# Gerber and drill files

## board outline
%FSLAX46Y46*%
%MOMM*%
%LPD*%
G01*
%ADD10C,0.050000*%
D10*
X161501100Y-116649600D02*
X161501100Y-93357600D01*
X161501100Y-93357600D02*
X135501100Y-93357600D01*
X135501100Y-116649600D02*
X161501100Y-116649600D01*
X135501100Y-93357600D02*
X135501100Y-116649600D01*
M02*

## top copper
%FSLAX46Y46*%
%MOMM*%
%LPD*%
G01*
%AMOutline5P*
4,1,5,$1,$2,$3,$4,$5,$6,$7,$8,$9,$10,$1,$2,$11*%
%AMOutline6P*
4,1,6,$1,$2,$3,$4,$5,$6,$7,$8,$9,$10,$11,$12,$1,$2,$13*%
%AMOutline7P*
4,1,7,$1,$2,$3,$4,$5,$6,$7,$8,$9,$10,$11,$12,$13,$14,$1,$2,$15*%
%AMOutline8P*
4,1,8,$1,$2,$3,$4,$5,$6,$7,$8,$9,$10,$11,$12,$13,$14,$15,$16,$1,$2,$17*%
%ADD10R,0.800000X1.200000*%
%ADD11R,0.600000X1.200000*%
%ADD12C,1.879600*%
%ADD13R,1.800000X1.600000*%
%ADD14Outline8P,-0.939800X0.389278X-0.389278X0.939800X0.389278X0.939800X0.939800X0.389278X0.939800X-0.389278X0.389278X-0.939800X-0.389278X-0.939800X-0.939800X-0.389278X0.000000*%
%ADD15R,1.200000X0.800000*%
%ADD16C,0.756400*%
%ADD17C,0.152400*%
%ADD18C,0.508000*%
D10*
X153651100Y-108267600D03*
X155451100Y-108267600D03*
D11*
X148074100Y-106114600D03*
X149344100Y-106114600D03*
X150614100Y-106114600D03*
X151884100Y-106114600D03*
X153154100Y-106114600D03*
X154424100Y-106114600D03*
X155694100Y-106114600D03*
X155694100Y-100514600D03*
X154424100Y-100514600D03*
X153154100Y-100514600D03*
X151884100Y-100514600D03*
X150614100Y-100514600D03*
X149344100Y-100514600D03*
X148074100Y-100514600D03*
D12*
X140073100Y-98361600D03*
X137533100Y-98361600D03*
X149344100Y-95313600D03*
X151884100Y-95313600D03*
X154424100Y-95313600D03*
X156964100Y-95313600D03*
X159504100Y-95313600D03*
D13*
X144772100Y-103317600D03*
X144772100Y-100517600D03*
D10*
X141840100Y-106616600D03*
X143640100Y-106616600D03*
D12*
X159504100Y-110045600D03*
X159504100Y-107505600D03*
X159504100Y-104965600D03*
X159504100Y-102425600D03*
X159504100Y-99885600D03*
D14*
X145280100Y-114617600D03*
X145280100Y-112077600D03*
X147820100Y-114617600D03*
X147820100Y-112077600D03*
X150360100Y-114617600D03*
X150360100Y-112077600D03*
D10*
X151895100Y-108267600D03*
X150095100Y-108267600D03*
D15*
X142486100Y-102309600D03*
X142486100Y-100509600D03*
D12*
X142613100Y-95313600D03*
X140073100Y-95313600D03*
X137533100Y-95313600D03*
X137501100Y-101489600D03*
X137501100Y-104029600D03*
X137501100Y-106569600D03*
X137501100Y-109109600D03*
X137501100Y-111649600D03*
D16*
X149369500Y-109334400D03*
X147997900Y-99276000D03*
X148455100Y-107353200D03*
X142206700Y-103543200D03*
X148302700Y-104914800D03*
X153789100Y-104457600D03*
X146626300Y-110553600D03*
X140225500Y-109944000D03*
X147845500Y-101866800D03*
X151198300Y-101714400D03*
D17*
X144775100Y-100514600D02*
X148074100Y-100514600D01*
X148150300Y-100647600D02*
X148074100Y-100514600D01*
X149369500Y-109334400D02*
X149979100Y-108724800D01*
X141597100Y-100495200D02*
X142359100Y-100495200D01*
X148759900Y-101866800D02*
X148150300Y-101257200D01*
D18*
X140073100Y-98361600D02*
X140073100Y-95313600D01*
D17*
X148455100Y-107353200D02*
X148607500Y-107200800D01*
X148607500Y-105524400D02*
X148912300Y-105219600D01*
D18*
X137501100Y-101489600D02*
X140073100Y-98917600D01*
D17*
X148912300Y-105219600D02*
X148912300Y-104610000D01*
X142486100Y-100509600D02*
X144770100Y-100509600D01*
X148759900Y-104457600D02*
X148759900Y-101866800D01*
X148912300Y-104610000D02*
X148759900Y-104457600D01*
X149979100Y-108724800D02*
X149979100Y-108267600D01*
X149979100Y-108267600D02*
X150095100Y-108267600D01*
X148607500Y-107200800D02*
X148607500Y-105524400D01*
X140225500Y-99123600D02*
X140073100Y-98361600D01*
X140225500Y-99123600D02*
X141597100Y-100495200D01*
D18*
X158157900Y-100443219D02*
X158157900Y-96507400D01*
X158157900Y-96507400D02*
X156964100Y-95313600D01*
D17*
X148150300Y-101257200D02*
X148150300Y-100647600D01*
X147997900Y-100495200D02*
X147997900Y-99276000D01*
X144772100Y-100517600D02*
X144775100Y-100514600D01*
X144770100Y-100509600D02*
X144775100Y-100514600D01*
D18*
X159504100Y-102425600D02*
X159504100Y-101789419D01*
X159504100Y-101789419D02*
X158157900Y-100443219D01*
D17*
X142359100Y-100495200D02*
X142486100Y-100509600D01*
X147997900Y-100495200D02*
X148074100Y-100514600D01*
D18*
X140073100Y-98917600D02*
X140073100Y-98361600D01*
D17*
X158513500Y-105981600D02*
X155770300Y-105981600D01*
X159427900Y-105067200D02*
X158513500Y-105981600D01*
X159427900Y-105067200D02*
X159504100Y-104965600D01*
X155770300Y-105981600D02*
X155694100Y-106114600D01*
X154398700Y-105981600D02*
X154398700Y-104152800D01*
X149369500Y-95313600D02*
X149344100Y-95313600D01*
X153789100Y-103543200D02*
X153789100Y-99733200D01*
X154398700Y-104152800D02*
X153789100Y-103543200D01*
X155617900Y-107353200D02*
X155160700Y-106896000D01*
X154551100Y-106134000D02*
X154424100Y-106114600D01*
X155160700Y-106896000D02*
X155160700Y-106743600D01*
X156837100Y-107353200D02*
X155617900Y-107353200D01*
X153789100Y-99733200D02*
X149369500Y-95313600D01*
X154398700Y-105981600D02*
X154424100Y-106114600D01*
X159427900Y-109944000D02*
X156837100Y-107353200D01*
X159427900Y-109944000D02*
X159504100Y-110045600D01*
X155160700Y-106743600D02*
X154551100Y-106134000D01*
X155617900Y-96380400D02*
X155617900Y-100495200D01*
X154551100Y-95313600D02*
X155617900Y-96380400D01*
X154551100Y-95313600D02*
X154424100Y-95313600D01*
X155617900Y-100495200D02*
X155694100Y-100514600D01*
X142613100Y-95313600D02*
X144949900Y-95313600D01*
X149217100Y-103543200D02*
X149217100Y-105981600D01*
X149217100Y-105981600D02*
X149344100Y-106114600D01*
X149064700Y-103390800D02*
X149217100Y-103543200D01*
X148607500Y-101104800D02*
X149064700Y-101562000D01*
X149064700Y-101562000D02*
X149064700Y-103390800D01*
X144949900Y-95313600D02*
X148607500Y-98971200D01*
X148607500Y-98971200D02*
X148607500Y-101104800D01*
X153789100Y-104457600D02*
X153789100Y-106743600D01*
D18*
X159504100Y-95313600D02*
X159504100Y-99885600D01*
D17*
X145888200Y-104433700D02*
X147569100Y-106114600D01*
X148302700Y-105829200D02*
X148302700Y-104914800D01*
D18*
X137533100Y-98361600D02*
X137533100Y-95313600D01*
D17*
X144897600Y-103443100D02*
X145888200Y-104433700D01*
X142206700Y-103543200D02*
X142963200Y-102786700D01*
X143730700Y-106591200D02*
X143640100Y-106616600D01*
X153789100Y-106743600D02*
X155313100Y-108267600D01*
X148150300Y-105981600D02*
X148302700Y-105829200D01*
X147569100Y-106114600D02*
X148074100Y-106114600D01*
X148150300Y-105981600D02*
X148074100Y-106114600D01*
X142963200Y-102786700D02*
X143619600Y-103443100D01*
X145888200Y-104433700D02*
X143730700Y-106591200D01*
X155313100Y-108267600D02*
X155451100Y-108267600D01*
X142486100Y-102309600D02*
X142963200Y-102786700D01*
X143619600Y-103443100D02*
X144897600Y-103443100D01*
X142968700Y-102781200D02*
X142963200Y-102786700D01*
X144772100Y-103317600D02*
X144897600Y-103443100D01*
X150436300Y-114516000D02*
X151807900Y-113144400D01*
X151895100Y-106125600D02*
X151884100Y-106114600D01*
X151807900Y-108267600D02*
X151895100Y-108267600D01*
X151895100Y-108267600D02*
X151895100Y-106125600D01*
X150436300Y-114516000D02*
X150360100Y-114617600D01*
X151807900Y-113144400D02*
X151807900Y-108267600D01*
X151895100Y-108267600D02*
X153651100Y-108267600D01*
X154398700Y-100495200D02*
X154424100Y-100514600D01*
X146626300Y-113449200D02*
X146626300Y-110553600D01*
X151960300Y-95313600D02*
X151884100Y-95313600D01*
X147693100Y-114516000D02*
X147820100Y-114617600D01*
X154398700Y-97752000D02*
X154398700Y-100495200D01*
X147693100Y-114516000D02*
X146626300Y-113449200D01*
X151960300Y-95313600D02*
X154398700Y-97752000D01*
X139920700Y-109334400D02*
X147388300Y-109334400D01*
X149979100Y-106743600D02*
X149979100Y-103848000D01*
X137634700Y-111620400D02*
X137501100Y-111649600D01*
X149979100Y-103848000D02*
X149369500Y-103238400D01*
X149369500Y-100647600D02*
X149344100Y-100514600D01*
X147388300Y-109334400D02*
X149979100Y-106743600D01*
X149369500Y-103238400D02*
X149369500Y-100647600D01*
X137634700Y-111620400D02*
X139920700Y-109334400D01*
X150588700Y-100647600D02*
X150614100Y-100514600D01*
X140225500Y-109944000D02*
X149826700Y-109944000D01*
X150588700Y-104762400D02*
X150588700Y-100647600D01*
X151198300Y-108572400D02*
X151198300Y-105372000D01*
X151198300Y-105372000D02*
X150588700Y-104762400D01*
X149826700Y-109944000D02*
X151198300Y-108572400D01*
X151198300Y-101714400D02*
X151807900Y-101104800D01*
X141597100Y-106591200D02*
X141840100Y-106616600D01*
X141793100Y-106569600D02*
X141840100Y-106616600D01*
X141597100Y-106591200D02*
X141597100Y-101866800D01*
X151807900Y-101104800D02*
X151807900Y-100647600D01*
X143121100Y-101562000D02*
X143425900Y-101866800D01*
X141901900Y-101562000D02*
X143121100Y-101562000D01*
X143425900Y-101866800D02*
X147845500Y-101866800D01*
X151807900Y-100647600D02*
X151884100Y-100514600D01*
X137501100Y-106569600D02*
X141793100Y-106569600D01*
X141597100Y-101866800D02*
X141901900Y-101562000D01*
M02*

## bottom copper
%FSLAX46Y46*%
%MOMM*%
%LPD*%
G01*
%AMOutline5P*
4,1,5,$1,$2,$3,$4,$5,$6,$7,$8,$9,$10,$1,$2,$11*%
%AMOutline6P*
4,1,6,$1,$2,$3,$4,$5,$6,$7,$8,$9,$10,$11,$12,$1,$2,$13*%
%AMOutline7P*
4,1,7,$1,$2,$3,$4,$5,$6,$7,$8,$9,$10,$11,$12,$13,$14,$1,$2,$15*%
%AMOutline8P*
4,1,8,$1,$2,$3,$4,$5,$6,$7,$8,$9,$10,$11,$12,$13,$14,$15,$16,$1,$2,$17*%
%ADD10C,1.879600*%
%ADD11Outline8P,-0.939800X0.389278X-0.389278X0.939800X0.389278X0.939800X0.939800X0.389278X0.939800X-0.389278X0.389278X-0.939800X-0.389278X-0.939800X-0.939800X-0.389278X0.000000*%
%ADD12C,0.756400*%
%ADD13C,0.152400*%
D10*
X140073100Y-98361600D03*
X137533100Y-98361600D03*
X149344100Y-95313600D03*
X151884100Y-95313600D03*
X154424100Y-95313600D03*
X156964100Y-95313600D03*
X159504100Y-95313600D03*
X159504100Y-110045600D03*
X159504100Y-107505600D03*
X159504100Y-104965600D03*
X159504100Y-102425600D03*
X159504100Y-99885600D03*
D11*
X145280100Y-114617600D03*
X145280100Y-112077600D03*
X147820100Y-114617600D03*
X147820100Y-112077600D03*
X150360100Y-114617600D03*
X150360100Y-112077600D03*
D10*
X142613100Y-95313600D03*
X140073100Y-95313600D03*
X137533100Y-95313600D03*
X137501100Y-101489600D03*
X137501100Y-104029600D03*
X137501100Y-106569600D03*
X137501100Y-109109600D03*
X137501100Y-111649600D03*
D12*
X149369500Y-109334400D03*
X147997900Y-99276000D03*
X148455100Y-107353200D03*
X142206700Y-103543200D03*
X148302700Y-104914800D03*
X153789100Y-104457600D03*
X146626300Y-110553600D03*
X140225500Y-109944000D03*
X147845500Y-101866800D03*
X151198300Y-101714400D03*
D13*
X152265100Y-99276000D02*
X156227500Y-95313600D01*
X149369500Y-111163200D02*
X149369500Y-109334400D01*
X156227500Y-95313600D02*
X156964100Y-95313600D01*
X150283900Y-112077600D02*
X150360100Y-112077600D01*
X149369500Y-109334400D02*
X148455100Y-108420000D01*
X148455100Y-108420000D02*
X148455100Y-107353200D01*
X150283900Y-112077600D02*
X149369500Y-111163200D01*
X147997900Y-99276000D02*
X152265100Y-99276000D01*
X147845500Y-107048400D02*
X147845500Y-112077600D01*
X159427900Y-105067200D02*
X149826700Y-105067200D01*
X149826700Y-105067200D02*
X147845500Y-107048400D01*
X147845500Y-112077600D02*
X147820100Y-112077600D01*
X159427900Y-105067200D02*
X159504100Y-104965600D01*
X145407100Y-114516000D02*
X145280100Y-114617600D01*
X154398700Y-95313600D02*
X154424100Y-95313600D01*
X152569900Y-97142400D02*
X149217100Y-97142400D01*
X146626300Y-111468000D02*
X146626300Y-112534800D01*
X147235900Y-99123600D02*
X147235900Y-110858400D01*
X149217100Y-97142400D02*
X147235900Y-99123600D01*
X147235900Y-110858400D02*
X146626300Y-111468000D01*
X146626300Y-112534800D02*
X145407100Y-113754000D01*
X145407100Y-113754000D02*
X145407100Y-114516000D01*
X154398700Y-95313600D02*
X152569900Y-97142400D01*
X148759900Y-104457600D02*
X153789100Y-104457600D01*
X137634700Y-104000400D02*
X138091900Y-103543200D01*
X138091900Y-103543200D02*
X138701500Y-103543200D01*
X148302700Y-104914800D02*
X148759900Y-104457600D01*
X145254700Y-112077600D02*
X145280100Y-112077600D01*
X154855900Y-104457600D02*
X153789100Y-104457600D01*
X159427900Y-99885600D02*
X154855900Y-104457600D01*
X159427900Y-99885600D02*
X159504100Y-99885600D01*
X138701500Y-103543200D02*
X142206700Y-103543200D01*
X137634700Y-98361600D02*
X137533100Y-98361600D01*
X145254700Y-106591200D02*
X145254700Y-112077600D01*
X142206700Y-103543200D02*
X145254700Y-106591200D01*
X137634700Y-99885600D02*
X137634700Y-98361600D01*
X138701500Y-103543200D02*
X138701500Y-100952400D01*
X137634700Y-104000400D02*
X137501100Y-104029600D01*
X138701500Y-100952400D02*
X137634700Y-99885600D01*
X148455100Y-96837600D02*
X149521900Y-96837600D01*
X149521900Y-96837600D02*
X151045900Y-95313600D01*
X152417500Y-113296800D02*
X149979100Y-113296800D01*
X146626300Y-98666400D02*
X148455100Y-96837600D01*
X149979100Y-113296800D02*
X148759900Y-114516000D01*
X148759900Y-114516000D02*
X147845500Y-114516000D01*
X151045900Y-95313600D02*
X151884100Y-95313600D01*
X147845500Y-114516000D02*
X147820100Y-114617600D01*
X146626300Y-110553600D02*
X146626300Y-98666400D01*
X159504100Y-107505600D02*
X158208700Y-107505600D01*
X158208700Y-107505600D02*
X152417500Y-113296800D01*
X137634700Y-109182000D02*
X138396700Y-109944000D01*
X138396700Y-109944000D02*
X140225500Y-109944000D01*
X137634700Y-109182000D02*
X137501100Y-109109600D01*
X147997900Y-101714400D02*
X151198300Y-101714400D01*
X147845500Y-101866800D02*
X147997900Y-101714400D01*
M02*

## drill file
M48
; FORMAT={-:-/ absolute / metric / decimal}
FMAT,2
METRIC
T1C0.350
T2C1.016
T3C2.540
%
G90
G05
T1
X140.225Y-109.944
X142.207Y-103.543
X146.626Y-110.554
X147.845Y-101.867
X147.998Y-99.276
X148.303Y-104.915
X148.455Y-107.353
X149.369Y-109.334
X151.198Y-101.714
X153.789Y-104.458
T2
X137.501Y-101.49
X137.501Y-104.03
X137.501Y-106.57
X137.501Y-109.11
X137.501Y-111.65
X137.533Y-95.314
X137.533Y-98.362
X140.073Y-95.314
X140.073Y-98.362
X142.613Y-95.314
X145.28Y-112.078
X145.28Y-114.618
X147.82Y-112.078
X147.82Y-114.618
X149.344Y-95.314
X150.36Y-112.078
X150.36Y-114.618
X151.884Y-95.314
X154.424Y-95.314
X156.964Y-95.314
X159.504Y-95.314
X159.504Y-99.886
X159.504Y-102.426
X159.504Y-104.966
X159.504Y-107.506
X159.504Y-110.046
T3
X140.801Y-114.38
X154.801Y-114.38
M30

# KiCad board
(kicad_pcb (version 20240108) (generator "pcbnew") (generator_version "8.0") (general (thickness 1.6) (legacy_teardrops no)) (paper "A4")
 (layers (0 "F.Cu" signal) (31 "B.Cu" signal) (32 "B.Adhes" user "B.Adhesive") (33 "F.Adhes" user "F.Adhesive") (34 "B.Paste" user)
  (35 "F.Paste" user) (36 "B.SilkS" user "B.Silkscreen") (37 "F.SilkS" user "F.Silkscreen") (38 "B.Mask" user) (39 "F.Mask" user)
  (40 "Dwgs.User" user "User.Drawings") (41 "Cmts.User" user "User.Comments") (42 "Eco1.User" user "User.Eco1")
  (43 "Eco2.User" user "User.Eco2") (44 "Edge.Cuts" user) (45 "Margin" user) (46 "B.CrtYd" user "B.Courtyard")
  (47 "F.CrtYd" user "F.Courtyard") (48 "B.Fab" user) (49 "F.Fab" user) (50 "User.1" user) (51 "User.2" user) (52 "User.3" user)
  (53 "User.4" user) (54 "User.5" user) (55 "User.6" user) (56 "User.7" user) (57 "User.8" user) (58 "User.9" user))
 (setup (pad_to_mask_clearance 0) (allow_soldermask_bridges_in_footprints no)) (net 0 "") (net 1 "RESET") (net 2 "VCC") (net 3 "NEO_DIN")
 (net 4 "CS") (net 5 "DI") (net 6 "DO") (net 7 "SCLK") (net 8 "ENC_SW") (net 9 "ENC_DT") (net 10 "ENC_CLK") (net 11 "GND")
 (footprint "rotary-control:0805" (layer "F.Cu") (at 154.5511 108.2676)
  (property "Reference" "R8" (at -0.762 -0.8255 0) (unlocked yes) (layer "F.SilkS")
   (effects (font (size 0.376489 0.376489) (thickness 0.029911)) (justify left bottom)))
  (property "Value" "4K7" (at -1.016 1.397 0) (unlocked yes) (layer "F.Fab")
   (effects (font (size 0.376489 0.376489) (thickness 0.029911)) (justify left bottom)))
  (pad "1" smd rect (at -0.9 0) (size 0.8 1.2) (layers "F.Cu" "F.Paste" "F.Mask") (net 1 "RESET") (solder_mask_margin 0.1016)
   (thermal_bridge_angle 0))
  (pad "2" smd rect (at 0.9 0) (size 0.8 1.2) (layers "F.Cu" "F.Paste" "F.Mask") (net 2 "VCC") (solder_mask_margin 0.1016)
   (thermal_bridge_angle 0)))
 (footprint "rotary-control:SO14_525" (layer "F.Cu") (at 151.2491 103.3146)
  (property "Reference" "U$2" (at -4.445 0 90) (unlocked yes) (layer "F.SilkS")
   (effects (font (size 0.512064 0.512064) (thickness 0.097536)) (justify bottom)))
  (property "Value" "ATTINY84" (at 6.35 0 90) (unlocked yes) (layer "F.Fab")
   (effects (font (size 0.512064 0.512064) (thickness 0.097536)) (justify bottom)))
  (pad "1" smd rect (at -3.175 2.8) (size 0.6 1.2) (layers "F.Cu" "F.Paste" "F.Mask") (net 2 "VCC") (solder_mask_margin 0.1016)
   (thermal_bridge_angle 0))
  (pad "2" smd rect (at -1.905 2.8) (size 0.6 1.2) (layers "F.Cu" "F.Paste" "F.Mask") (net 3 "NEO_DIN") (solder_mask_margin 0.1016)
   (thermal_bridge_angle 0))
  (pad "3" smd rect (at -0.635 2.8) (size 0.6 1.2) (layers "F.Cu" "F.Paste" "F.Mask") (solder_mask_margin 0.1016) (thermal_bridge_angle 0))
  (pad "4" smd rect (at 0.635 2.8) (size 0.6 1.2) (layers "F.Cu" "F.Paste" "F.Mask") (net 1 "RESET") (solder_mask_margin 0.1016)
   (thermal_bridge_angle 0))
  (pad "5" smd rect (at 1.905 2.8) (size 0.6 1.2) (layers "F.Cu" "F.Paste" "F.Mask") (solder_mask_margin 0.1016) (thermal_bridge_angle 0))
  (pad "6" smd rect (at 3.175 2.8) (size 0.6 1.2) (layers "F.Cu" "F.Paste" "F.Mask") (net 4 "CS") (solder_mask_margin 0.1016)
   (thermal_bridge_angle 0))
  (pad "7" smd rect (at 4.445 2.8) (size 0.6 1.2) (layers "F.Cu" "F.Paste" "F.Mask") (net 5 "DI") (solder_mask_margin 0.1016)
   (thermal_bridge_angle 0))
  (pad "8" smd rect (at 4.445 -2.8) (size 0.6 1.2) (layers "F.Cu" "F.Paste" "F.Mask") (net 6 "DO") (solder_mask_margin 0.1016)
   (thermal_bridge_angle 0))
  (pad "9" smd rect (at 3.175 -2.8) (size 0.6 1.2) (layers "F.Cu" "F.Paste" "F.Mask") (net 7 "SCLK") (solder_mask_margin 0.1016)
   (thermal_bridge_angle 0))
  (pad "10" smd rect (at 1.905 -2.8) (size 0.6 1.2) (layers "F.Cu" "F.Paste" "F.Mask") (solder_mask_margin 0.1016) (thermal_bridge_angle 0))
  (pad "11" smd rect (at 0.635 -2.8) (size 0.6 1.2) (layers "F.Cu" "F.Paste" "F.Mask") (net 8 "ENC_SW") (solder_mask_margin 0.1016)
   (thermal_bridge_angle 0))
  (pad "12" smd rect (at -0.635 -2.8) (size 0.6 1.2) (layers "F.Cu" "F.Paste" "F.Mask") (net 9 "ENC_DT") (solder_mask_margin 0.1016)
   (thermal_bridge_angle 0))
  (pad "13" smd rect (at -1.905 -2.8) (size 0.6 1.2) (layers "F.Cu" "F.Paste" "F.Mask") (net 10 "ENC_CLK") (solder_mask_margin 0.1016)
   (thermal_bridge_angle 0))
  (pad "14" smd rect (at -3.175 -2.8) (size 0.6 1.2) (layers "F.Cu" "F.Paste" "F.Mask") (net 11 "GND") (solder_mask_margin 0.1016)
   (thermal_bridge_angle 0)))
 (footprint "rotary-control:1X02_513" (layer "F.Cu") (at 140.0731 98.3616 180)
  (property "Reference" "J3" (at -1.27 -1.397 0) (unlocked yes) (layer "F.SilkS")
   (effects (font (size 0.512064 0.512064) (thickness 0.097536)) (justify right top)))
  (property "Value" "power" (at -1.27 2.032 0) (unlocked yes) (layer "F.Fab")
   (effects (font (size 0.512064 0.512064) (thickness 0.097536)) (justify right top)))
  (pad "1" thru_hole circle (at 0 0 270) (size 1.8796 1.8796) (drill 1.016) (layers "*.Cu" "*.Mask") (remove_unused_layers no)
   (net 11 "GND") (solder_mask_margin 0.1016) (thermal_bridge_angle 0))
  (pad "2" thru_hole circle (at 2.54 0 270) (size 1.8796 1.8796) (drill 1.016) (layers "*.Cu" "*.Mask") (remove_unused_layers no)
   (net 2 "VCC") (solder_mask_margin 0.1016) (thermal_bridge_angle 0)))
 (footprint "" (layer "F.Cu") (at 140.8011 114.3796)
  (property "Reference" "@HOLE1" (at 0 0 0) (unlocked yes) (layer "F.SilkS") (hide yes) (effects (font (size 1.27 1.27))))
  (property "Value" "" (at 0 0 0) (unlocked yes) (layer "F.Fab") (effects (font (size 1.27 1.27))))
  (pad "" np_thru_hole circle (at 0 0) (size 2.54 2.54) (drill 2.54) (layers "*.Cu" "*.Mask")))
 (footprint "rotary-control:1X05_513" (layer "F.Cu") (at 149.3441 95.3136)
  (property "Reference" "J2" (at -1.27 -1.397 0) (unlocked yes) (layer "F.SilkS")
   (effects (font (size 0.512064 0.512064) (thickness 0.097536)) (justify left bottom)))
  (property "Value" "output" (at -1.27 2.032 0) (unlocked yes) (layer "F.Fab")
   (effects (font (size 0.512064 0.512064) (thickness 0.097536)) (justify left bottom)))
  (pad "1" thru_hole circle (at 0 0 90) (size 1.8796 1.8796) (drill 1.016) (layers "*.Cu" "*.Mask") (remove_unused_layers no) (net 4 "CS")
   (solder_mask_margin 0.1016) (thermal_bridge_angle 0))
  (pad "2" thru_hole circle (at 2.54 0 90) (size 1.8796 1.8796) (drill 1.016) (layers "*.Cu" "*.Mask") (remove_unused_layers no)
   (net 7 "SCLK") (solder_mask_margin 0.1016) (thermal_bridge_angle 0))
  (pad "3" thru_hole circle (at 5.08 0 90) (size 1.8796 1.8796) (drill 1.016) (layers "*.Cu" "*.Mask") (remove_unused_layers no)
   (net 6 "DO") (solder_mask_margin 0.1016) (thermal_bridge_angle 0))
  (pad "4" thru_hole circle (at 7.62 0 90) (size 1.8796 1.8796) (drill 1.016) (layers "*.Cu" "*.Mask") (remove_unused_layers no)
   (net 11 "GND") (solder_mask_margin 0.1016) (thermal_bridge_angle 0))
  (pad "5" thru_hole circle (at 10.16 0 90) (size 1.8796 1.8796) (drill 1.016) (layers "*.Cu" "*.Mask") (remove_unused_layers no)
   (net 2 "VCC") (solder_mask_margin 0.1016) (thermal_bridge_angle 0)))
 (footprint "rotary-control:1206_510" (layer "F.Cu") (at 144.7721 101.9176 90)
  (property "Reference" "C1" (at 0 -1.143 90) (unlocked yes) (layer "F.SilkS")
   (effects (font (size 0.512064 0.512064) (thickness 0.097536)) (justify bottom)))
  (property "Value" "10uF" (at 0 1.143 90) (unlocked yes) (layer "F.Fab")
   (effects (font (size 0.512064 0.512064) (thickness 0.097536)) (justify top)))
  (pad "1" smd rect (at -1.4 0 90) (size 1.6 1.8) (layers "F.Cu" "F.Paste" "F.Mask") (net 2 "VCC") (solder_mask_margin 0.1016)
   (thermal_bridge_angle 0))
  (pad "2" smd rect (at 1.4 0 90) (size 1.6 1.8) (layers "F.Cu" "F.Paste" "F.Mask") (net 11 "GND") (solder_mask_margin 0.1016)
   (thermal_bridge_angle 0)))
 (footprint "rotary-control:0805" (layer "F.Cu") (at 142.7401 106.6166)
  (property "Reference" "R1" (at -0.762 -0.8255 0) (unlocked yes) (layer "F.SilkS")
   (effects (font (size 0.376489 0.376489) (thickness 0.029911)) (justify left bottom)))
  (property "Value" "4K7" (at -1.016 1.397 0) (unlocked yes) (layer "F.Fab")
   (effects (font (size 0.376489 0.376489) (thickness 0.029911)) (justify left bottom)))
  (pad "1" smd rect (at -0.9 0) (size 0.8 1.2) (layers "F.Cu" "F.Paste" "F.Mask") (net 8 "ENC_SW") (solder_mask_margin 0.1016)
   (thermal_bridge_angle 0))
  (pad "2" smd rect (at 0.9 0) (size 0.8 1.2) (layers "F.Cu" "F.Paste" "F.Mask") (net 2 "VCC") (solder_mask_margin 0.1016)
   (thermal_bridge_angle 0)))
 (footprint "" (layer "F.Cu") (at 154.8011 114.3796)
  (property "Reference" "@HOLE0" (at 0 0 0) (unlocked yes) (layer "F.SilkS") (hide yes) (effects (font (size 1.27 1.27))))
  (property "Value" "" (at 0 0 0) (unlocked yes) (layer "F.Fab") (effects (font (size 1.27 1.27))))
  (pad "" np_thru_hole circle (at 0 0) (size 2.54 2.54) (drill 2.54) (layers "*.Cu" "*.Mask")))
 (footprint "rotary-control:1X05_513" (layer "F.Cu") (at 159.5041 110.0456 90)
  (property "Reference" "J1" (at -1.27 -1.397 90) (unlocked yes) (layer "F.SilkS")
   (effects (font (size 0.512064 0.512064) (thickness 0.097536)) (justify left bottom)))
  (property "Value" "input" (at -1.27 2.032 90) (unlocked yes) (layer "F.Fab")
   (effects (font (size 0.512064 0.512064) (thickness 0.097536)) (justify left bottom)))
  (pad "1" thru_hole circle (at 0 0 180) (size 1.8796 1.8796) (drill 1.016) (layers "*.Cu" "*.Mask") (remove_unused_layers no) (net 4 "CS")
   (solder_mask_margin 0.1016) (thermal_bridge_angle 0))
  (pad "2" thru_hole circle (at 2.54 0 180) (size 1.8796 1.8796) (drill 1.016) (layers "*.Cu" "*.Mask") (remove_unused_layers no)
   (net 7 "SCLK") (solder_mask_margin 0.1016) (thermal_bridge_angle 0))
  (pad "3" thru_hole circle (at 5.08 0 180) (size 1.8796 1.8796) (drill 1.016) (layers "*.Cu" "*.Mask") (remove_unused_layers no)
   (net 5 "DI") (solder_mask_margin 0.1016) (thermal_bridge_angle 0))
  (pad "4" thru_hole circle (at 7.62 0 180) (size 1.8796 1.8796) (drill 1.016) (layers "*.Cu" "*.Mask") (remove_unused_layers no)
   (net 11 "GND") (solder_mask_margin 0.1016) (thermal_bridge_angle 0))
  (pad "5" thru_hole circle (at 10.16 0 180) (size 1.8796 1.8796) (drill 1.016) (layers "*.Cu" "*.Mask") (remove_unused_layers no)
   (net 2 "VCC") (solder_mask_margin 0.1016) (thermal_bridge_angle 0)))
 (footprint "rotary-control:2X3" (layer "F.Cu") (at 145.2801 114.6176)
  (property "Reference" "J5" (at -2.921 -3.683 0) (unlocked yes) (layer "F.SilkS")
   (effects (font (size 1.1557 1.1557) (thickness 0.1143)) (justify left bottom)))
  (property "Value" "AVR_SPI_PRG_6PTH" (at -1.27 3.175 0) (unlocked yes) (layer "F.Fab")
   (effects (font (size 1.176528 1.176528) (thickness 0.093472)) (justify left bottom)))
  (pad "1" thru_hole roundrect (at 0 0) (size 1.8796 1.8796) (drill 1.016) (layers "*.Cu" "*.Mask") (remove_unused_layers no)
   (roundrect_rratio 0.25) (chamfer_ratio 0.2928932188) (chamfer top_left top_right bottom_left bottom_right) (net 6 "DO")
   (solder_mask_margin 0.1016) (thermal_bridge_angle 0))
  (pad "2" thru_hole roundrect (at 0 -2.54) (size 1.8796 1.8796) (drill 1.016) (layers "*.Cu" "*.Mask") (remove_unused_layers no)
   (roundrect_rratio 0.25) (chamfer_ratio 0.2928932188) (chamfer top_left top_right bottom_left bottom_right) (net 2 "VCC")
   (solder_mask_margin 0.1016) (thermal_bridge_angle 0))
  (pad "3" thru_hole roundrect (at 2.54 0) (size 1.8796 1.8796) (drill 1.016) (layers "*.Cu" "*.Mask") (remove_unused_layers no)
   (roundrect_rratio 0.25) (chamfer_ratio 0.2928932188) (chamfer top_left top_right bottom_left bottom_right) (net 7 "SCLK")
   (solder_mask_margin 0.1016) (thermal_bridge_angle 0))
  (pad "4" thru_hole roundrect (at 2.54 -2.54) (size 1.8796 1.8796) (drill 1.016) (layers "*.Cu" "*.Mask") (remove_unused_layers no)
   (roundrect_rratio 0.25) (chamfer_ratio 0.2928932188) (chamfer top_left top_right bottom_left bottom_right) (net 5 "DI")
   (solder_mask_margin 0.1016) (thermal_bridge_angle 0))
  (pad "5" thru_hole roundrect (at 5.08 0) (size 1.8796 1.8796) (drill 1.016) (layers "*.Cu" "*.Mask") (remove_unused_layers no)
   (roundrect_rratio 0.25) (chamfer_ratio 0.2928932188) (chamfer top_left top_right bottom_left bottom_right) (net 1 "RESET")
   (solder_mask_margin 0.1016) (thermal_bridge_angle 0))
  (pad "6" thru_hole roundrect (at 5.08 -2.54) (size 1.8796 1.8796) (drill 1.016) (layers "*.Cu" "*.Mask") (remove_unused_layers no)
   (roundrect_rratio 0.25) (chamfer_ratio 0.2928932188) (chamfer top_left top_right bottom_left bottom_right) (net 11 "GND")
   (solder_mask_margin 0.1016) (thermal_bridge_angle 0)))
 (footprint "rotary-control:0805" (layer "F.Cu") (at 150.9951 108.2676 180)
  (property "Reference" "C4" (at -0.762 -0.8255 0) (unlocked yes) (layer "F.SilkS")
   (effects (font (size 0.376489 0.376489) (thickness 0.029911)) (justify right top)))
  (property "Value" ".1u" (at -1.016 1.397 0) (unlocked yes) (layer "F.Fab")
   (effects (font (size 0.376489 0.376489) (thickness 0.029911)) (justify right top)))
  (pad "1" smd rect (at -0.9 0 180) (size 0.8 1.2) (layers "F.Cu" "F.Paste" "F.Mask") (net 1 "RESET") (solder_mask_margin 0.1016)
   (thermal_bridge_angle 0))
  (pad "2" smd rect (at 0.9 0 180) (size 0.8 1.2) (layers "F.Cu" "F.Paste" "F.Mask") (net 11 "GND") (solder_mask_margin 0.1016)
   (thermal_bridge_angle 0)))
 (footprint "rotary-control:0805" (layer "F.Cu") (at 142.4861 101.4096 90)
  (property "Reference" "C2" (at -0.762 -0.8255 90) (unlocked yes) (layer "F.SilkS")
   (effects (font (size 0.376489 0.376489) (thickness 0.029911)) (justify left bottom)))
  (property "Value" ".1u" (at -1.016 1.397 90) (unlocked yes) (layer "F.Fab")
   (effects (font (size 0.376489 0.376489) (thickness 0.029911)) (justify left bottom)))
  (pad "1" smd rect (at -0.9 0 90) (size 0.8 1.2) (layers "F.Cu" "F.Paste" "F.Mask") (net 2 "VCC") (solder_mask_margin 0.1016)
   (thermal_bridge_angle 0))
  (pad "2" smd rect (at 0.9 0 90) (size 0.8 1.2) (layers "F.Cu" "F.Paste" "F.Mask") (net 11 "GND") (solder_mask_margin 0.1016)
   (thermal_bridge_angle 0)))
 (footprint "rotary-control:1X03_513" (layer "B.Cu") (at 142.6131 95.3136 180)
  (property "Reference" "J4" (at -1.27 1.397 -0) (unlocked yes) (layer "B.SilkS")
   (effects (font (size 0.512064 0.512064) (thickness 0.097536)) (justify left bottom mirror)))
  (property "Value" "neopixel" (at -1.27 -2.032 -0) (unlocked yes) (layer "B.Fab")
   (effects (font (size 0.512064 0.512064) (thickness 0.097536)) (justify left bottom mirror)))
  (pad "1" thru_hole circle (at 0 0 90) (size 1.8796 1.8796) (drill 1.016) (layers "*.Cu" "*.Mask") (remove_unused_layers no)
   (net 3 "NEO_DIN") (solder_mask_margin 0.1016) (thermal_bridge_angle 0))
  (pad "2" thru_hole circle (at 2.54 0 90) (size 1.8796 1.8796) (drill 1.016) (layers "*.Cu" "*.Mask") (remove_unused_layers no)
   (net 11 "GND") (solder_mask_margin 0.1016) (thermal_bridge_angle 0))
  (pad "3" thru_hole circle (at 5.08 0 90) (size 1.8796 1.8796) (drill 1.016) (layers "*.Cu" "*.Mask") (remove_unused_layers no)
   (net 2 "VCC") (solder_mask_margin 0.1016) (thermal_bridge_angle 0)))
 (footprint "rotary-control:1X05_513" (layer "B.Cu") (at 137.5011 101.4896 -90)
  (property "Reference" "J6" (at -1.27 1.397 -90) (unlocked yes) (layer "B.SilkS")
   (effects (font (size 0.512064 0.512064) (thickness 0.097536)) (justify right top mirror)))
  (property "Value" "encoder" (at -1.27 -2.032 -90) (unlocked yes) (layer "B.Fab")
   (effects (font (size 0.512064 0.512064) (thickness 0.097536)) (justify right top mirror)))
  (pad "1" thru_hole circle (at 0 0 180) (size 1.8796 1.8796) (drill 1.016) (layers "*.Cu" "*.Mask") (remove_unused_layers no)
   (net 11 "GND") (solder_mask_margin 0.1016) (thermal_bridge_angle 0))
  (pad "2" thru_hole circle (at 2.54 0 180) (size 1.8796 1.8796) (drill 1.016) (layers "*.Cu" "*.Mask") (remove_unused_layers no)
   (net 2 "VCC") (solder_mask_margin 0.1016) (thermal_bridge_angle 0))
  (pad "3" thru_hole circle (at 5.08 0 180) (size 1.8796 1.8796) (drill 1.016) (layers "*.Cu" "*.Mask") (remove_unused_layers no)
   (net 8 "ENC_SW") (solder_mask_margin 0.1016) (thermal_bridge_angle 0))
  (pad "4" thru_hole circle (at 7.62 0 180) (size 1.8796 1.8796) (drill 1.016) (layers "*.Cu" "*.Mask") (remove_unused_layers no)
   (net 9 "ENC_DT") (solder_mask_margin 0.1016) (thermal_bridge_angle 0))
  (pad "5" thru_hole circle (at 10.16 0 180) (size 1.8796 1.8796) (drill 1.016) (layers "*.Cu" "*.Mask") (remove_unused_layers no)
   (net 10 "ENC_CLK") (solder_mask_margin 0.1016) (thermal_bridge_angle 0)))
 (gr_line (start 161.5011 116.6496) (end 161.5011 93.3576) (stroke (width 0.05) (type solid)) (layer "Edge.Cuts"))
 (gr_line (start 161.5011 93.3576) (end 135.5011 93.3576) (stroke (width 0.05) (type solid)) (layer "Edge.Cuts"))
 (gr_line (start 135.5011 116.6496) (end 161.5011 116.6496) (stroke (width 0.05) (type solid)) (layer "Edge.Cuts"))
 (gr_line (start 135.5011 93.3576) (end 135.5011 116.6496) (stroke (width 0.05) (type solid)) (layer "Edge.Cuts"))
 (segment (start 144.7751 100.5146) (end 148.0741 100.5146) (width 0.1524) (layer "F.Cu") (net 11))
 (segment (start 148.1503 100.6476) (end 148.0741 100.5146) (width 0.1524) (layer "F.Cu") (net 11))
 (segment (start 149.3695 109.3344) (end 149.9791 108.7248) (width 0.1524) (layer "F.Cu") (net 11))
 (segment (start 141.5971 100.4952) (end 142.3591 100.4952) (width 0.1524) (layer "F.Cu") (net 11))
 (segment (start 148.7599 101.8668) (end 148.1503 101.2572) (width 0.1524) (layer "F.Cu") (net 11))
 (segment (start 140.0731 98.3616) (end 140.0731 95.3136) (width 0.508) (layer "F.Cu") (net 11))
 (segment (start 148.4551 107.3532) (end 148.6075 107.2008) (width 0.1524) (layer "F.Cu") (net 11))
 (segment (start 148.6075 105.5244) (end 148.9123 105.2196) (width 0.1524) (layer "F.Cu") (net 11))
 (segment (start 137.5011 101.4896) (end 140.0731 98.9176) (width 0.508) (layer "F.Cu") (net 11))
 (segment (start 148.9123 105.2196) (end 148.9123 104.61) (width 0.1524) (layer "F.Cu") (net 11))
 (segment (start 142.4861 100.5096) (end 144.7701 100.5096) (width 0.1524) (layer "F.Cu") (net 11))
 (segment (start 148.7599 104.4576) (end 148.7599 101.8668) (width 0.1524) (layer "F.Cu") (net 11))
 (segment (start 148.9123 104.61) (end 148.7599 104.4576) (width 0.1524) (layer "F.Cu") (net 11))
 (segment (start 149.9791 108.7248) (end 149.9791 108.2676) (width 0.1524) (layer "F.Cu") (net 11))
 (segment (start 149.9791 108.2676) (end 150.0951 108.2676) (width 0.1524) (layer "F.Cu") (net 11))
 (segment (start 148.6075 107.2008) (end 148.6075 105.5244) (width 0.1524) (layer "F.Cu") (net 11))
 (segment (start 140.2255 99.1236) (end 140.0731 98.3616) (width 0.1524) (layer "F.Cu") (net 11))
 (segment (start 140.2255 99.1236) (end 141.5971 100.4952) (width 0.1524) (layer "F.Cu") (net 11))
 (segment (start 158.1579 100.443219) (end 158.1579 96.5074) (width 0.508) (layer "F.Cu") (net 11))
 (segment (start 158.1579 96.5074) (end 156.9641 95.3136) (width 0.508) (layer "F.Cu") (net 11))
 (segment (start 148.1503 101.2572) (end 148.1503 100.6476) (width 0.1524) (layer "F.Cu") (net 11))
 (segment (start 147.9979 100.4952) (end 147.9979 99.276) (width 0.1524) (layer "F.Cu") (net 11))
 (segment (start 144.7721 100.5176) (end 144.7751 100.5146) (width 0.1524) (layer "F.Cu") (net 11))
 (segment (start 144.7701 100.5096) (end 144.7751 100.5146) (width 0.1524) (layer "F.Cu") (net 11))
 (segment (start 159.5041 102.4256) (end 159.5041 101.789419) (width 0.508) (layer "F.Cu") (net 11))
 (segment (start 159.5041 101.789419) (end 158.1579 100.443219) (width 0.508) (layer "F.Cu") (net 11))
 (segment (start 142.3591 100.4952) (end 142.4861 100.5096) (width 0.1524) (layer "F.Cu") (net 11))
 (segment (start 147.9979 100.4952) (end 148.0741 100.5146) (width 0.1524) (layer "F.Cu") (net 11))
 (segment (start 140.0731 98.9176) (end 140.0731 98.3616) (width 0.508) (layer "F.Cu") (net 11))
 (via (at 149.3695 109.3344) (size 0.7564) (drill 0.35) (layers "F.Cu" "B.Cu") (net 11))
 (via (at 147.9979 99.276) (size 0.7564) (drill 0.35) (layers "F.Cu" "B.Cu") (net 11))
 (via (at 148.4551 107.3532) (size 0.7564) (drill 0.35) (layers "F.Cu" "B.Cu") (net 11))
 (segment (start 152.2651 99.276) (end 156.2275 95.3136) (width 0.1524) (layer "B.Cu") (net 11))
 (segment (start 149.3695 111.1632) (end 149.3695 109.3344) (width 0.1524) (layer "B.Cu") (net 11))
 (segment (start 156.2275 95.3136) (end 156.9641 95.3136) (width 0.1524) (layer "B.Cu") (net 11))
 (segment (start 150.2839 112.0776) (end 150.3601 112.0776) (width 0.1524) (layer "B.Cu") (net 11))
 (segment (start 149.3695 109.3344) (end 148.4551 108.42) (width 0.1524) (layer "B.Cu") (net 11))
 (segment (start 148.4551 108.42) (end 148.4551 107.3532) (width 0.1524) (layer "B.Cu") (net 11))
 (segment (start 150.2839 112.0776) (end 149.3695 111.1632) (width 0.1524) (layer "B.Cu") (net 11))
 (segment (start 147.9979 99.276) (end 152.2651 99.276) (width 0.1524) (layer "B.Cu") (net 11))
 (segment (start 158.5135 105.9816) (end 155.7703 105.9816) (width 0.1524) (layer "F.Cu") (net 5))
 (segment (start 159.4279 105.0672) (end 158.5135 105.9816) (width 0.1524) (layer "F.Cu") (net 5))
 (segment (start 159.4279 105.0672) (end 159.5041 104.9656) (width 0.1524) (layer "F.Cu") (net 5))
 (segment (start 155.7703 105.9816) (end 155.6941 106.1146) (width 0.1524) (layer "F.Cu") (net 5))
 (segment (start 147.8455 107.0484) (end 147.8455 112.0776) (width 0.1524) (layer "B.Cu") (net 5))
 (segment (start 159.4279 105.0672) (end 149.8267 105.0672) (width 0.1524) (layer "B.Cu") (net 5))
 (segment (start 149.8267 105.0672) (end 147.8455 107.0484) (width 0.1524) (layer "B.Cu") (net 5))
 (segment (start 147.8455 112.0776) (end 147.8201 112.0776) (width 0.1524) (layer "B.Cu") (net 5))
 (segment (start 159.4279 105.0672) (end 159.5041 104.9656) (width 0.1524) (layer "B.Cu") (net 5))
 (segment (start 154.3987 105.9816) (end 154.3987 104.1528) (width 0.1524) (layer "F.Cu") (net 4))
 (segment (start 149.3695 95.3136) (end 149.3441 95.3136) (width 0.1524) (layer "F.Cu") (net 4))
 (segment (start 153.7891 103.5432) (end 153.7891 99.7332) (width 0.1524) (layer "F.Cu") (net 4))
 (segment (start 154.3987 104.1528) (end 153.7891 103.5432) (width 0.1524) (layer "F.Cu") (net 4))
 (segment (start 155.6179 107.3532) (end 155.1607 106.896) (width 0.1524) (layer "F.Cu") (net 4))
 (segment (start 154.5511 106.134) (end 154.4241 106.1146) (width 0.1524) (layer "F.Cu") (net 4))
 (segment (start 155.1607 106.896) (end 155.1607 106.7436) (width 0.1524) (layer "F.Cu") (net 4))
 (segment (start 156.8371 107.3532) (end 155.6179 107.3532) (width 0.1524) (layer "F.Cu") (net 4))
 (segment (start 153.7891 99.7332) (end 149.3695 95.3136) (width 0.1524) (layer "F.Cu") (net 4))
 (segment (start 154.3987 105.9816) (end 154.4241 106.1146) (width 0.1524) (layer "F.Cu") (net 4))
 (segment (start 159.4279 109.944) (end 156.8371 107.3532) (width 0.1524) (layer "F.Cu") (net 4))
 (segment (start 159.4279 109.944) (end 159.5041 110.0456) (width 0.1524) (layer "F.Cu") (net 4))
 (segment (start 155.1607 106.7436) (end 154.5511 106.134) (width 0.1524) (layer "F.Cu") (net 4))
 (segment (start 155.6179 96.3804) (end 155.6179 100.4952) (width 0.1524) (layer "F.Cu") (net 6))
 (segment (start 154.5511 95.3136) (end 155.6179 96.3804) (width 0.1524) (layer "F.Cu") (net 6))
 (segment (start 154.5511 95.3136) (end 154.4241 95.3136) (width 0.1524) (layer "F.Cu") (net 6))
 (segment (start 155.6179 100.4952) (end 155.6941 100.5146) (width 0.1524) (layer "F.Cu") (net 6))
 (segment (start 145.4071 114.516) (end 145.2801 114.6176) (width 0.1524) (layer "B.Cu") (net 6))
 (segment (start 154.3987 95.3136) (end 154.4241 95.3136) (width 0.1524) (layer "B.Cu") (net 6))
 (segment (start 152.5699 97.1424) (end 149.2171 97.1424) (width 0.1524) (layer "B.Cu") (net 6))
 (segment (start 146.6263 111.468) (end 146.6263 112.5348) (width 0.1524) (layer "B.Cu") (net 6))
 (segment (start 147.2359 99.1236) (end 147.2359 110.8584) (width 0.1524) (layer "B.Cu") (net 6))
 (segment (start 149.2171 97.1424) (end 147.2359 99.1236) (width 0.1524) (layer "B.Cu") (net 6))
 (segment (start 147.2359 110.8584) (end 146.6263 111.468) (width 0.1524) (layer "B.Cu") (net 6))
 (segment (start 146.6263 112.5348) (end 145.4071 113.754) (width 0.1524) (layer "B.Cu") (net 6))
 (segment (start 145.4071 113.754) (end 145.4071 114.516) (width 0.1524) (layer "B.Cu") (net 6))
 (segment (start 154.3987 95.3136) (end 152.5699 97.1424) (width 0.1524) (layer "B.Cu") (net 6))
 (segment (start 142.6131 95.3136) (end 144.9499 95.3136) (width 0.1524) (layer "F.Cu") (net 3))
 (segment (start 149.2171 103.5432) (end 149.2171 105.9816) (width 0.1524) (layer "F.Cu") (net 3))
 (segment (start 149.2171 105.9816) (end 149.3441 106.1146) (width 0.1524) (layer "F.Cu") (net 3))
 (segment (start 149.0647 103.3908) (end 149.2171 103.5432) (width 0.1524) (layer "F.Cu") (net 3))
 (segment (start 148.6075 101.1048) (end 149.0647 101.562) (width 0.1524) (layer "F.Cu") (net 3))
 (segment (start 149.0647 101.562) (end 149.0647 103.3908) (width 0.1524) (layer "F.Cu") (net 3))
 (segment (start 144.9499 95.3136) (end 148.6075 98.9712) (width 0.1524) (layer "F.Cu") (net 3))
 (segment (start 148.6075 98.9712) (end 148.6075 101.1048) (width 0.1524) (layer "F.Cu") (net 3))
 (segment (start 153.7891 104.4576) (end 153.7891 106.7436) (width 0.1524) (layer "F.Cu") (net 2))
 (segment (start 159.5041 95.3136) (end 159.5041 99.8856) (width 0.508) (layer "F.Cu") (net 2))
 (segment (start 145.8882 104.4337) (end 147.5691 106.1146) (width 0.1524) (layer "F.Cu") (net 2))
 (segment (start 148.3027 105.8292) (end 148.3027 104.9148) (width 0.1524) (layer "F.Cu") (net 2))
 (segment (start 137.5331 98.3616) (end 137.5331 95.3136) (width 0.508) (layer "F.Cu") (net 2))
 (segment (start 144.8976 103.4431) (end 145.8882 104.4337) (width 0.1524) (layer "F.Cu") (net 2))
 (segment (start 142.2067 103.5432) (end 142.9632 102.7867) (width 0.1524) (layer "F.Cu") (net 2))
 (segment (start 143.7307 106.5912) (end 143.6401 106.6166) (width 0.1524) (layer "F.Cu") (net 2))
 (segment (start 153.7891 106.7436) (end 155.3131 108.2676) (width 0.1524) (layer "F.Cu") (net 2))
 (segment (start 148.1503 105.9816) (end 148.3027 105.8292) (width 0.1524) (layer "F.Cu") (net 2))
 (segment (start 147.5691 106.1146) (end 148.0741 106.1146) (width 0.1524) (layer "F.Cu") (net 2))
 (segment (start 148.1503 105.9816) (end 148.0741 106.1146) (width 0.1524) (layer "F.Cu") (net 2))
 (segment (start 142.9632 102.7867) (end 143.6196 103.4431) (width 0.1524) (layer "F.Cu") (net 2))
 (segment (start 145.8882 104.4337) (end 143.7307 106.5912) (width 0.1524) (layer "F.Cu") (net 2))
 (segment (start 155.3131 108.2676) (end 155.4511 108.2676) (width 0.1524) (layer "F.Cu") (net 2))
 (segment (start 142.4861 102.3096) (end 142.9632 102.7867) (width 0.1524) (layer "F.Cu") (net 2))
 (segment (start 143.6196 103.4431) (end 144.8976 103.4431) (width 0.1524) (layer "F.Cu") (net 2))
 (segment (start 142.9687 102.7812) (end 142.9632 102.7867) (width 0.1524) (layer "F.Cu") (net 2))
 (segment (start 144.7721 103.3176) (end 144.8976 103.4431) (width 0.1524) (layer "F.Cu") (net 2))
 (via (at 142.2067 103.5432) (size 0.7564) (drill 0.35) (layers "F.Cu" "B.Cu") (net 2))
 (via (at 148.3027 104.9148) (size 0.7564) (drill 0.35) (layers "F.Cu" "B.Cu") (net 2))
 (via (at 153.7891 104.4576) (size 0.7564) (drill 0.35) (layers "F.Cu" "B.Cu") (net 2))
 (segment (start 148.7599 104.4576) (end 153.7891 104.4576) (width 0.1524) (layer "B.Cu") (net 2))
 (segment (start 137.6347 104.0004) (end 138.0919 103.5432) (width 0.1524) (layer "B.Cu") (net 2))
 (segment (start 138.0919 103.5432) (end 138.7015 103.5432) (width 0.1524) (layer "B.Cu") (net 2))
 (segment (start 148.3027 104.9148) (end 148.7599 104.4576) (width 0.1524) (layer "B.Cu") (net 2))
 (segment (start 145.2547 112.0776) (end 145.2801 112.0776) (width 0.1524) (layer "B.Cu") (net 2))
 (segment (start 154.8559 104.4576) (end 153.7891 104.4576) (width 0.1524) (layer "B.Cu") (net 2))
 (segment (start 159.4279 99.8856) (end 154.8559 104.4576) (width 0.1524) (layer "B.Cu") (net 2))
 (segment (start 159.4279 99.8856) (end 159.5041 99.8856) (width 0.1524) (layer "B.Cu") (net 2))
 (segment (start 138.7015 103.5432) (end 142.2067 103.5432) (width 0.1524) (layer "B.Cu") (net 2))
 (segment (start 137.6347 98.3616) (end 137.5331 98.3616) (width 0.1524) (layer "B.Cu") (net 2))
 (segment (start 145.2547 106.5912) (end 145.2547 112.0776) (width 0.1524) (layer "B.Cu") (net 2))
 (segment (start 142.2067 103.5432) (end 145.2547 106.5912) (width 0.1524) (layer "B.Cu") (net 2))
 (segment (start 137.6347 99.8856) (end 137.6347 98.3616) (width 0.1524) (layer "B.Cu") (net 2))
 (segment (start 138.7015 103.5432) (end 138.7015 100.9524) (width 0.1524) (layer "B.Cu") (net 2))
 (segment (start 137.6347 104.0004) (end 137.5011 104.0296) (width 0.1524) (layer "B.Cu") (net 2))
 (segment (start 138.7015 100.9524) (end 137.6347 99.8856) (width 0.1524) (layer "B.Cu") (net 2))
 (segment (start 150.4363 114.516) (end 151.8079 113.1444) (width 0.1524) (layer "F.Cu") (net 1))
 (segment (start 151.8951 106.1256) (end 151.8841 106.1146) (width 0.1524) (layer "F.Cu") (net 1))
 (segment (start 151.8079 108.2676) (end 151.8951 108.2676) (width 0.1524) (layer "F.Cu") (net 1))
 (segment (start 151.8951 108.2676) (end 151.8951 106.1256) (width 0.1524) (layer "F.Cu") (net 1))
 (segment (start 150.4363 114.516) (end 150.3601 114.6176) (width 0.1524) (layer "F.Cu") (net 1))
 (segment (start 151.8079 113.1444) (end 151.8079 108.2676) (width 0.1524) (layer "F.Cu") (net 1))
 (segment (start 151.8951 108.2676) (end 153.6511 108.2676) (width 0.1524) (layer "F.Cu") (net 1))
 (segment (start 154.3987 100.4952) (end 154.4241 100.5146) (width 0.1524) (layer "F.Cu") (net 7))
 (segment (start 146.6263 113.4492) (end 146.6263 110.5536) (width 0.1524) (layer "F.Cu") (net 7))
 (segment (start 151.9603 95.3136) (end 151.8841 95.3136) (width 0.1524) (layer "F.Cu") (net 7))
 (segment (start 147.6931 114.516) (end 147.8201 114.6176) (width 0.1524) (layer "F.Cu") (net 7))
 (segment (start 154.3987 97.752) (end 154.3987 100.4952) (width 0.1524) (layer "F.Cu") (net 7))
 (segment (start 147.6931 114.516) (end 146.6263 113.4492) (width 0.1524) (layer "F.Cu") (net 7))
 (segment (start 151.9603 95.3136) (end 154.3987 97.752) (width 0.1524) (layer "F.Cu") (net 7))
 (via (at 146.6263 110.5536) (size 0.7564) (drill 0.35) (layers "F.Cu" "B.Cu") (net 7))
 (segment (start 148.4551 96.8376) (end 149.5219 96.8376) (width 0.1524) (layer "B.Cu") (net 7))
 (segment (start 149.5219 96.8376) (end 151.0459 95.3136) (width 0.1524) (layer "B.Cu") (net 7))
 (segment (start 152.4175 113.2968) (end 149.9791 113.2968) (width 0.1524) (layer "B.Cu") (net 7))
 (segment (start 146.6263 98.6664) (end 148.4551 96.8376) (width 0.1524) (layer "B.Cu") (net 7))
 (segment (start 149.9791 113.2968) (end 148.7599 114.516) (width 0.1524) (layer "B.Cu") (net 7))
 (segment (start 148.7599 114.516) (end 147.8455 114.516) (width 0.1524) (layer "B.Cu") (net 7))
 (segment (start 151.0459 95.3136) (end 151.8841 95.3136) (width 0.1524) (layer "B.Cu") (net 7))
 (segment (start 147.8455 114.516) (end 147.8201 114.6176) (width 0.1524) (layer "B.Cu") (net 7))
 (segment (start 146.6263 110.5536) (end 146.6263 98.6664) (width 0.1524) (layer "B.Cu") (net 7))
 (segment (start 159.5041 107.5056) (end 158.2087 107.5056) (width 0.1524) (layer "B.Cu") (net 7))
 (segment (start 158.2087 107.5056) (end 152.4175 113.2968) (width 0.1524) (layer "B.Cu") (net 7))
 (segment (start 139.9207 109.3344) (end 147.3883 109.3344) (width 0.1524) (layer "F.Cu") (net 10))
 (segment (start 149.9791 106.7436) (end 149.9791 103.848) (width 0.1524) (layer "F.Cu") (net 10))
 (segment (start 137.6347 111.6204) (end 137.5011 111.6496) (width 0.1524) (layer "F.Cu") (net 10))
 (segment (start 149.9791 103.848) (end 149.3695 103.2384) (width 0.1524) (layer "F.Cu") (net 10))
 (segment (start 149.3695 100.6476) (end 149.3441 100.5146) (width 0.1524) (layer "F.Cu") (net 10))
 (segment (start 147.3883 109.3344) (end 149.9791 106.7436) (width 0.1524) (layer "F.Cu") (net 10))
 (segment (start 149.3695 103.2384) (end 149.3695 100.6476) (width 0.1524) (layer "F.Cu") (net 10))
 (segment (start 137.6347 111.6204) (end 139.9207 109.3344) (width 0.1524) (layer "F.Cu") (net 10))
 (segment (start 150.5887 100.6476) (end 150.6141 100.5146) (width 0.1524) (layer "F.Cu") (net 9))
 (segment (start 140.2255 109.944) (end 149.8267 109.944) (width 0.1524) (layer "F.Cu") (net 9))
 (segment (start 150.5887 104.7624) (end 150.5887 100.6476) (width 0.1524) (layer "F.Cu") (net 9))
 (segment (start 151.1983 108.5724) (end 151.1983 105.372) (width 0.1524) (layer "F.Cu") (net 9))
 (segment (start 151.1983 105.372) (end 150.5887 104.7624) (width 0.1524) (layer "F.Cu") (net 9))
 (segment (start 149.8267 109.944) (end 151.1983 108.5724) (width 0.1524) (layer "F.Cu") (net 9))
 (via (at 140.2255 109.944) (size 0.7564) (drill 0.35) (layers "F.Cu" "B.Cu") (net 9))
 (segment (start 137.6347 109.182) (end 138.3967 109.944) (width 0.1524) (layer "B.Cu") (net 9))
 (segment (start 138.3967 109.944) (end 140.2255 109.944) (width 0.1524) (layer "B.Cu") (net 9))
 (segment (start 137.6347 109.182) (end 137.5011 109.1096) (width 0.1524) (layer "B.Cu") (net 9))
 (segment (start 151.1983 101.7144) (end 151.8079 101.1048) (width 0.1524) (layer "F.Cu") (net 8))
 (segment (start 141.5971 106.5912) (end 141.8401 106.6166) (width 0.1524) (layer "F.Cu") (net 8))
 (segment (start 141.7931 106.5696) (end 141.8401 106.6166) (width 0.1524) (layer "F.Cu") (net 8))
 (segment (start 141.5971 106.5912) (end 141.5971 101.8668) (width 0.1524) (layer "F.Cu") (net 8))
 (segment (start 151.8079 101.1048) (end 151.8079 100.6476) (width 0.1524) (layer "F.Cu") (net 8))
 (segment (start 143.1211 101.562) (end 143.4259 101.8668) (width 0.1524) (layer "F.Cu") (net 8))
 (segment (start 141.9019 101.562) (end 143.1211 101.562) (width 0.1524) (layer "F.Cu") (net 8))
 (segment (start 143.4259 101.8668) (end 147.8455 101.8668) (width 0.1524) (layer "F.Cu") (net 8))
 (segment (start 151.8079 100.6476) (end 151.8841 100.5146) (width 0.1524) (layer "F.Cu") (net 8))
 (segment (start 137.5011 106.5696) (end 141.7931 106.5696) (width 0.1524) (layer "F.Cu") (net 8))
 (segment (start 141.5971 101.8668) (end 141.9019 101.562) (width 0.1524) (layer "F.Cu") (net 8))
 (via (at 147.8455 101.8668) (size 0.7564) (drill 0.35) (layers "F.Cu" "B.Cu") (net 8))
 (via (at 151.1983 101.7144) (size 0.7564) (drill 0.35) (layers "F.Cu" "B.Cu") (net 8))
 (segment (start 147.9979 101.7144) (end 151.1983 101.7144) (width 0.1524) (layer "B.Cu") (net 8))
 (segment (start 147.8455 101.8668) (end 147.9979 101.7144) (width 0.1524) (layer "B.Cu") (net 8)))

